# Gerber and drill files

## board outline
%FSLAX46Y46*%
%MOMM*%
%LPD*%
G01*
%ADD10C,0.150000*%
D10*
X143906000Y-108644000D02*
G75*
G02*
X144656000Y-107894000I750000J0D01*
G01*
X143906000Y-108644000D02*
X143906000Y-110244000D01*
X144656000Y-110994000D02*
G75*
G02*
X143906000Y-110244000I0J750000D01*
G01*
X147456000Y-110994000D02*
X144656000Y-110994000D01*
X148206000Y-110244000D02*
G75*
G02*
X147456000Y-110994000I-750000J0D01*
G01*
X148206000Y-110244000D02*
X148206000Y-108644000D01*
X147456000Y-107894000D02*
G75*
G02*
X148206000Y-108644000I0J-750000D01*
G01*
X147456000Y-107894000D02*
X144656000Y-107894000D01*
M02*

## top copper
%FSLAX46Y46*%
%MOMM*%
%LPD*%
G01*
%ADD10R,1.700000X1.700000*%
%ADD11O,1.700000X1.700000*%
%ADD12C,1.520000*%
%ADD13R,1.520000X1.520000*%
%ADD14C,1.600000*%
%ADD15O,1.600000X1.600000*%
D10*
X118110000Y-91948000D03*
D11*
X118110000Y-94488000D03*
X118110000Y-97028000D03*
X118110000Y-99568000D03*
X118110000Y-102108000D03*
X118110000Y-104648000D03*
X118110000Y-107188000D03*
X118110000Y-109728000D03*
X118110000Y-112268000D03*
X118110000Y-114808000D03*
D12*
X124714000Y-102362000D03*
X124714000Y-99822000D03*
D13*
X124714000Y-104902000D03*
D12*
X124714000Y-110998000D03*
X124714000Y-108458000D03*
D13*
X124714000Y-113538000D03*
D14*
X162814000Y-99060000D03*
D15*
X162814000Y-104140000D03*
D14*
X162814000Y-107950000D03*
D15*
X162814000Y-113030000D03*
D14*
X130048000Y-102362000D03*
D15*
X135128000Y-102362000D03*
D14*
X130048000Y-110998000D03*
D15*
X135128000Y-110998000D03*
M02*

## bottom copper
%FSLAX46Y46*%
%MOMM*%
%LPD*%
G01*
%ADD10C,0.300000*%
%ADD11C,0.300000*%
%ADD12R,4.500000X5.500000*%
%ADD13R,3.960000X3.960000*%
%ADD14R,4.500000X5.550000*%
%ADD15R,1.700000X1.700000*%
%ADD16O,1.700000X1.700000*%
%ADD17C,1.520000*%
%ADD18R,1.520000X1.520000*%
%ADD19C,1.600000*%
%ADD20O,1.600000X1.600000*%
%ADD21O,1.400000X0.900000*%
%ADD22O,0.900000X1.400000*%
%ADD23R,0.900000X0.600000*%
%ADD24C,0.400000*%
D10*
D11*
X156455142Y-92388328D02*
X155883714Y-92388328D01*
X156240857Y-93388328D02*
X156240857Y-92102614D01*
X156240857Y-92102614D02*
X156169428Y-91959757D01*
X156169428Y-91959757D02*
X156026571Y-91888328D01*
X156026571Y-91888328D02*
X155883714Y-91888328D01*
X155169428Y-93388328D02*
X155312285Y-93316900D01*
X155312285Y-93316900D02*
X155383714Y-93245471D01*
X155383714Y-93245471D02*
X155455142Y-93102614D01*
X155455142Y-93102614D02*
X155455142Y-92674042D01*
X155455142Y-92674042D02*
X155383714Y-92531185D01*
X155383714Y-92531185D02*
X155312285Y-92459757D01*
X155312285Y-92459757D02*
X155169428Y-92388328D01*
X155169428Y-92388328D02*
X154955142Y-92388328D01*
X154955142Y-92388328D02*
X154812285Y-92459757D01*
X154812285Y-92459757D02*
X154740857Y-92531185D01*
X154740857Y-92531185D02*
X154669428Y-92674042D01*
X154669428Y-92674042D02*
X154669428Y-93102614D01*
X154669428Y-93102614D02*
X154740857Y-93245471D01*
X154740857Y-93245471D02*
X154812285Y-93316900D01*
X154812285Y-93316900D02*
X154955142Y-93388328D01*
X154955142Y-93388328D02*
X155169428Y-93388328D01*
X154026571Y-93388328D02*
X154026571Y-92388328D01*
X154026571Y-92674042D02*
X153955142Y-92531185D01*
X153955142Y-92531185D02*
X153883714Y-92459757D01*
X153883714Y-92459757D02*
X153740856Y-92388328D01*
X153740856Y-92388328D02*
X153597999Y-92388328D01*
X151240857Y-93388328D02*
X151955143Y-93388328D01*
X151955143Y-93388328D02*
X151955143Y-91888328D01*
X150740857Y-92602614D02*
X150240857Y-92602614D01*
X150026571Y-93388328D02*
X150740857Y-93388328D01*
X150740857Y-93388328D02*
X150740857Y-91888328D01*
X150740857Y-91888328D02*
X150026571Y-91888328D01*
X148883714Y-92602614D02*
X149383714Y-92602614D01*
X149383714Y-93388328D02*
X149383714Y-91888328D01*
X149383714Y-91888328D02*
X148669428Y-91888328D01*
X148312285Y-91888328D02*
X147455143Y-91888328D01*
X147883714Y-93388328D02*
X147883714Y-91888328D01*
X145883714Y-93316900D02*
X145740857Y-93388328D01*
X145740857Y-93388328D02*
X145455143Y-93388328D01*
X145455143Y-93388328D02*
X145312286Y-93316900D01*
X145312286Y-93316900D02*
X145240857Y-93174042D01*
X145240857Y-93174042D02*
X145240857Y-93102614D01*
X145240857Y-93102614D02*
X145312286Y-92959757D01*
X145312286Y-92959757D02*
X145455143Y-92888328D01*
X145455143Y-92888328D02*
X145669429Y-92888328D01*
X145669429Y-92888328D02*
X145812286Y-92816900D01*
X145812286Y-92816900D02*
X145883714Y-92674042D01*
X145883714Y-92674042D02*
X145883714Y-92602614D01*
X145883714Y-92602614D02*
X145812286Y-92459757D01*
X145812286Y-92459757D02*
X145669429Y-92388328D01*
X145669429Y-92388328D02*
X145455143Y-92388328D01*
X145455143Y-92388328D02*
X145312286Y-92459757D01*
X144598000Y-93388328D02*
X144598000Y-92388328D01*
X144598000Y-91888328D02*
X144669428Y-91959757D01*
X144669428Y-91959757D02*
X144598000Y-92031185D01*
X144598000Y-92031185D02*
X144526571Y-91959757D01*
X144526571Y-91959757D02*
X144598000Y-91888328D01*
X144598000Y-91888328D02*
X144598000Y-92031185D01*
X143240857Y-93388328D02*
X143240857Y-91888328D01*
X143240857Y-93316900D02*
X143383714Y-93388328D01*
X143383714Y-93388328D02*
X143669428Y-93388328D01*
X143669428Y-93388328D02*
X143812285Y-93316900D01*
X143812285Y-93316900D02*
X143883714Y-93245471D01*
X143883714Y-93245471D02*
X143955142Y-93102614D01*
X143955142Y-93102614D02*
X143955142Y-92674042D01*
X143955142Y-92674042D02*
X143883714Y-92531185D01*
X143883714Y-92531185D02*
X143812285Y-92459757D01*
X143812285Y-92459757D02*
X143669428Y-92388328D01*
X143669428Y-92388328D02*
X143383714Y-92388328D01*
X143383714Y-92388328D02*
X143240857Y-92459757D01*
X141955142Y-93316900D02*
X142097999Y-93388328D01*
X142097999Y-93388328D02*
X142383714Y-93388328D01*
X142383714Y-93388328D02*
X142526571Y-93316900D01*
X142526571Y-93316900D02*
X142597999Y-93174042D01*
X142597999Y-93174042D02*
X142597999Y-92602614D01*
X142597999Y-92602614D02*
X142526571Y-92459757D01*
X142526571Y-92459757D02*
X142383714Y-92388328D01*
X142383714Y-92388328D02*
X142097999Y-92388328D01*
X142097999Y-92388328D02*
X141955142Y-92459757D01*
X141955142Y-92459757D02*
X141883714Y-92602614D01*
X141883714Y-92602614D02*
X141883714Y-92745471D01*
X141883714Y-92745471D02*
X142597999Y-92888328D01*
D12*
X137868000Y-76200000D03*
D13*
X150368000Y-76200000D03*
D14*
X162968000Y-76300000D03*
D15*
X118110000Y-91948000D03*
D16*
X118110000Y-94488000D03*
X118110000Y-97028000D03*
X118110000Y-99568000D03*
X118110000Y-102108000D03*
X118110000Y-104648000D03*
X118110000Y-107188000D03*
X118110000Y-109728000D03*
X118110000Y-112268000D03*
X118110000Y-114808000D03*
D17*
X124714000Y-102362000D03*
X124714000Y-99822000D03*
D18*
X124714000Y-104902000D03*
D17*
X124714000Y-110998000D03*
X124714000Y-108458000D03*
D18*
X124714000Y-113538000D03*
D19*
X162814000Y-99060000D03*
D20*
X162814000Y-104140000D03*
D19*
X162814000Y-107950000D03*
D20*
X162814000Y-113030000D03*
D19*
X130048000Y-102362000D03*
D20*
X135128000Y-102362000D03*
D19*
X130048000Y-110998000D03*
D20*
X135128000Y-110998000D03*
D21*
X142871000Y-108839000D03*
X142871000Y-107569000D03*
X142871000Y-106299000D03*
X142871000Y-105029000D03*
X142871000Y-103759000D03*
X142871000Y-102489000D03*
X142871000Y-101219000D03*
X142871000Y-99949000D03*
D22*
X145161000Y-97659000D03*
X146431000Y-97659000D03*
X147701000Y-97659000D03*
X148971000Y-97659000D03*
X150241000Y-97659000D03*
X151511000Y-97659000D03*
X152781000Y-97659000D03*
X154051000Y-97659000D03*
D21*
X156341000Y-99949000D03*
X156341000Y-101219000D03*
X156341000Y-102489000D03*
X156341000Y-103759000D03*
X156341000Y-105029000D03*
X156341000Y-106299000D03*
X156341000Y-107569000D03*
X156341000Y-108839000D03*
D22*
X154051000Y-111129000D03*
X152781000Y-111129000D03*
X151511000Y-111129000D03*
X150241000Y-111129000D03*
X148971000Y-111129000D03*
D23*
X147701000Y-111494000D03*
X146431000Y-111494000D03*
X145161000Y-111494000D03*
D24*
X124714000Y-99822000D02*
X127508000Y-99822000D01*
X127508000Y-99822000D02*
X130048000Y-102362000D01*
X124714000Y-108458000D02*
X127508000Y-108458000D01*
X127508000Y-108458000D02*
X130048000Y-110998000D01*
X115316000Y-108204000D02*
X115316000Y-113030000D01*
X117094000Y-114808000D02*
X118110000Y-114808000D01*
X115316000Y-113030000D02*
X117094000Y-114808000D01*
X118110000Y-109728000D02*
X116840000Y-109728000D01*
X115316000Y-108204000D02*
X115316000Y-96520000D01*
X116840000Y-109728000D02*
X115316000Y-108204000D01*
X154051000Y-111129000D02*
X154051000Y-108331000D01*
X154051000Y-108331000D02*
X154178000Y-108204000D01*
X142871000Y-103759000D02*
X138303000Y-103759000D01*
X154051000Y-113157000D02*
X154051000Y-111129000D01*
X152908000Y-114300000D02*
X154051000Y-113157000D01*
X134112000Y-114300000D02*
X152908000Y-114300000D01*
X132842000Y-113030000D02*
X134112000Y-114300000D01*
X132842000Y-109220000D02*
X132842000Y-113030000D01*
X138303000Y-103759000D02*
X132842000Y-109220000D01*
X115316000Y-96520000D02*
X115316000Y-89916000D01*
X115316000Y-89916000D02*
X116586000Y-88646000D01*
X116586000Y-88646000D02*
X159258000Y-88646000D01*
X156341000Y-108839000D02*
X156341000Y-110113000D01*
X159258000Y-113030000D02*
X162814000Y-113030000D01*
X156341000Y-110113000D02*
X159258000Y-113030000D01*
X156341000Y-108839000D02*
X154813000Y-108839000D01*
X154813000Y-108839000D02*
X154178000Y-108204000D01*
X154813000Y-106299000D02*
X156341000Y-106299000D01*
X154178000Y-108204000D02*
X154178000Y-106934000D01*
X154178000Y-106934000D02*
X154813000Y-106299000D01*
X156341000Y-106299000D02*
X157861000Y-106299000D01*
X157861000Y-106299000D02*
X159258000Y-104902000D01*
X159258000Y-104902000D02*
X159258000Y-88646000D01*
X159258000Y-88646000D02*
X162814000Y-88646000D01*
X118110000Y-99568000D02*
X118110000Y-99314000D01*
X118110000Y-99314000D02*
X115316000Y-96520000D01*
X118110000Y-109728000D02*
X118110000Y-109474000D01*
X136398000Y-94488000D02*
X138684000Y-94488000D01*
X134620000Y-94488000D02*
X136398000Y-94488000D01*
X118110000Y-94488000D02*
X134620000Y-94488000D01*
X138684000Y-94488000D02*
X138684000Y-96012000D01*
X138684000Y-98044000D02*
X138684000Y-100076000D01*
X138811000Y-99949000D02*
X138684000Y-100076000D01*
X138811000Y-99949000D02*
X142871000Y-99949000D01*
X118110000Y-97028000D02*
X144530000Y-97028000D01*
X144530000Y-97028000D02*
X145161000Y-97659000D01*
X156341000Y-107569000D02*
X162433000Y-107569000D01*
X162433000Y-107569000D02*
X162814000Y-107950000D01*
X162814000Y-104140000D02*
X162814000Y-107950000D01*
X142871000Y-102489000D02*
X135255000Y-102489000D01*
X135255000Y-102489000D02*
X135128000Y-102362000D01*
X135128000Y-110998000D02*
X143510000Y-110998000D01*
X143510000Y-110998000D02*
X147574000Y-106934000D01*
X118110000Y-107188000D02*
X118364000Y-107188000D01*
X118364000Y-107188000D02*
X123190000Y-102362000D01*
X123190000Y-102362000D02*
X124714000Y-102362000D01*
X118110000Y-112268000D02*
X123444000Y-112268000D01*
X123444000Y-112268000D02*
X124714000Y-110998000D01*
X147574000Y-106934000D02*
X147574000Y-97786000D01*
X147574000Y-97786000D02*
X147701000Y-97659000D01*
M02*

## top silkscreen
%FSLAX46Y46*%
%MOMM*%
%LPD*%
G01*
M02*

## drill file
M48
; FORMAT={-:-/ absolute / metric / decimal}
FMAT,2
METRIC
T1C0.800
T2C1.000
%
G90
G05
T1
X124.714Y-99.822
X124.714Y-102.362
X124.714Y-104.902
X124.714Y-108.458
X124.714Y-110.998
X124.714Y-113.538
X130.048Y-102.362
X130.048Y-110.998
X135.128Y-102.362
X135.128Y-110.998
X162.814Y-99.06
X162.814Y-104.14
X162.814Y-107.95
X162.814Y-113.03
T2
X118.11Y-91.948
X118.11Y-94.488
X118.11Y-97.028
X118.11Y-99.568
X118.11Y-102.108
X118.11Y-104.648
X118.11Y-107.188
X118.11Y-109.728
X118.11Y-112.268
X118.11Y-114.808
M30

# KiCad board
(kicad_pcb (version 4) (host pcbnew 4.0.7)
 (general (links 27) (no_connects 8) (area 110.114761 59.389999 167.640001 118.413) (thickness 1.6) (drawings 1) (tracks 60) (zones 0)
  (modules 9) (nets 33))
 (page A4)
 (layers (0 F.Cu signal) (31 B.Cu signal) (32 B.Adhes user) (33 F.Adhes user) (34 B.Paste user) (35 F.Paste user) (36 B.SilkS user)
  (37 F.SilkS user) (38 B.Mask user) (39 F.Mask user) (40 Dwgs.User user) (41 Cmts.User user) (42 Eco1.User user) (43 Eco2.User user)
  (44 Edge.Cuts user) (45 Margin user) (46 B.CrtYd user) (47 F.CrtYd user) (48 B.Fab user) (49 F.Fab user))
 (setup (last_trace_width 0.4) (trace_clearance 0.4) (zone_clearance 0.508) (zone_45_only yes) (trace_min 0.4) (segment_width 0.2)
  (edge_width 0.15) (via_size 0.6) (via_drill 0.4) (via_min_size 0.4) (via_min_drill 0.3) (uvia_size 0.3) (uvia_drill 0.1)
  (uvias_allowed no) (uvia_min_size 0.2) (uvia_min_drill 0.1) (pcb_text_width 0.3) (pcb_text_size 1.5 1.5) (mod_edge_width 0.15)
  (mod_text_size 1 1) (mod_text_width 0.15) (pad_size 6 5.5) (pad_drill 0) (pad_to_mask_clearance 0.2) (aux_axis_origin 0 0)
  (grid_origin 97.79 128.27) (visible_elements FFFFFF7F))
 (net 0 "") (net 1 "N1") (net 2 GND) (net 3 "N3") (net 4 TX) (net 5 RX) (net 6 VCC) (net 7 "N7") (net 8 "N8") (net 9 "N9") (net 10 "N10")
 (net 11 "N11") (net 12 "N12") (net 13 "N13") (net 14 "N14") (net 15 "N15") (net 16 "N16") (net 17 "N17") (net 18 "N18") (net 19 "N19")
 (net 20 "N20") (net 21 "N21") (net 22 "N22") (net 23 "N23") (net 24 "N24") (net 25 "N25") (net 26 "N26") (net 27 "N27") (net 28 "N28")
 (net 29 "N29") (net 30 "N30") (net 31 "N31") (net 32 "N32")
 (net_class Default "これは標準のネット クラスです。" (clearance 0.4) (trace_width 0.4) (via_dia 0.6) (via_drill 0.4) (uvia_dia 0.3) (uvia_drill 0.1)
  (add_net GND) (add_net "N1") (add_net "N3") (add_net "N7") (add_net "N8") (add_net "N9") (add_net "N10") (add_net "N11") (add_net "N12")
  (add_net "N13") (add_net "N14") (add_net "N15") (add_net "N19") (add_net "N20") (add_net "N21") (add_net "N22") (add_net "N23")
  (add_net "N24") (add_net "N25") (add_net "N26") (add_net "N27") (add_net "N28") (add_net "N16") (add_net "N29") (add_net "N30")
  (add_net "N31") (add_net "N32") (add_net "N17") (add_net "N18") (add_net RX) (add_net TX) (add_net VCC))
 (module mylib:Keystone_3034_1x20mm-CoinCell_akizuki (layer B.Cu) (at 150.368 76.2)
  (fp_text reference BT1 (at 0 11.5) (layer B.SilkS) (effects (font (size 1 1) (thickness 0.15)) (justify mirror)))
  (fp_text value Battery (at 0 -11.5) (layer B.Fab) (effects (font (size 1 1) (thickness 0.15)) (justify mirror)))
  (pad 1 smd rect (at -12.5 0) (size 4.5 5.5) (layers B.Cu B.Paste B.Mask) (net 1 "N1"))
  (pad 2 smd rect (at 0 0) (size 3.96 3.96) (layers B.Cu B.Paste B.Mask) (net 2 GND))
  (pad 1 smd rect (at 12.6 0.1) (size 4.5 5.55) (layers B.Cu B.Paste B.Mask) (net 1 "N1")))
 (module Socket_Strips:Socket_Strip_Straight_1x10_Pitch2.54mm (layer B.Cu) (at 118.11 91.948 180)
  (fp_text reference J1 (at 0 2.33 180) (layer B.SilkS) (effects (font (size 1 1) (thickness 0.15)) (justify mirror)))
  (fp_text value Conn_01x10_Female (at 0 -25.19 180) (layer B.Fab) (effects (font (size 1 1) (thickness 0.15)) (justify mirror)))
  (pad 1 thru_hole rect (at 0 0 180) (size 1.7 1.7) (drill 1) (layers *.Cu *.Mask) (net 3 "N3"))
  (pad 2 thru_hole oval (at 0 -2.54 180) (size 1.7 1.7) (drill 1) (layers *.Cu *.Mask) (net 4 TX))
  (pad 3 thru_hole oval (at 0 -5.08 180) (size 1.7 1.7) (drill 1) (layers *.Cu *.Mask) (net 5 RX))
  (pad 4 thru_hole oval (at 0 -7.62 180) (size 1.7 1.7) (drill 1) (layers *.Cu *.Mask) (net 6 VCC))
  (pad 5 thru_hole oval (at 0 -10.16 180) (size 1.7 1.7) (drill 1) (layers *.Cu *.Mask) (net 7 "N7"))
  (pad 6 thru_hole oval (at 0 -12.7 180) (size 1.7 1.7) (drill 1) (layers *.Cu *.Mask) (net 2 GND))
  (pad 7 thru_hole oval (at 0 -15.24 180) (size 1.7 1.7) (drill 1) (layers *.Cu *.Mask) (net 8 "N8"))
  (pad 8 thru_hole oval (at 0 -17.78 180) (size 1.7 1.7) (drill 1) (layers *.Cu *.Mask) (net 6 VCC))
  (pad 9 thru_hole oval (at 0 -20.32 180) (size 1.7 1.7) (drill 1) (layers *.Cu *.Mask) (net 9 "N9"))
  (pad 10 thru_hole oval (at 0 -22.86 180) (size 1.7 1.7) (drill 1) (layers *.Cu *.Mask) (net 6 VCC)))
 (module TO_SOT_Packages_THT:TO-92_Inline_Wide (layer B.Cu) (at 124.714 104.902 90)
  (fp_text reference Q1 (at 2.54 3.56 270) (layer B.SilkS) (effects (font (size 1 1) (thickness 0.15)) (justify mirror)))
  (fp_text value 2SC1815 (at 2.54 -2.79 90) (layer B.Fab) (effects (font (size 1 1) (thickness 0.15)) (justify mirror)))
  (pad 2 thru_hole circle (at 2.54 0) (size 1.52 1.52) (drill 0.8) (layers *.Cu *.Mask) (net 8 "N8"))
  (pad 3 thru_hole circle (at 5.08 0) (size 1.52 1.52) (drill 0.8) (layers *.Cu *.Mask) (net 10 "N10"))
  (pad 1 thru_hole rect (at 0 0) (size 1.52 1.52) (drill 0.8) (layers *.Cu *.Mask) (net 2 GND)))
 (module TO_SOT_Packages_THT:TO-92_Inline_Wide (layer B.Cu) (at 124.714 113.538 90)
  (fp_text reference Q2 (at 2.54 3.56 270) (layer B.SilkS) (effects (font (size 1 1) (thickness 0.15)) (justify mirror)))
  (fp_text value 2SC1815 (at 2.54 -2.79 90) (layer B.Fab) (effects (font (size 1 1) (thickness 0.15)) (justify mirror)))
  (pad 2 thru_hole circle (at 2.54 0) (size 1.52 1.52) (drill 0.8) (layers *.Cu *.Mask) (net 9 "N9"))
  (pad 3 thru_hole circle (at 5.08 0) (size 1.52 1.52) (drill 0.8) (layers *.Cu *.Mask) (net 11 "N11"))
  (pad 1 thru_hole rect (at 0 0) (size 1.52 1.52) (drill 0.8) (layers *.Cu *.Mask) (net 2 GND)))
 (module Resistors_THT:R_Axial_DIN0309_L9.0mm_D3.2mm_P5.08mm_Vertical (layer B.Cu) (at 162.814 99.06 270)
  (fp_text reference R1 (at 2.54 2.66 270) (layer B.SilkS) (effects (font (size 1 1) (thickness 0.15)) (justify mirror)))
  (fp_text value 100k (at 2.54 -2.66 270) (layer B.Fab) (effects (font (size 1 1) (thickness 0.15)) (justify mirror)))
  (pad 1 thru_hole circle (at 0 0 270) (size 1.6 1.6) (drill 0.8) (layers *.Cu *.Mask) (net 2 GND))
  (pad 2 thru_hole oval (at 5.08 0 270) (size 1.6 1.6) (drill 0.8) (layers *.Cu *.Mask) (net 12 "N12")))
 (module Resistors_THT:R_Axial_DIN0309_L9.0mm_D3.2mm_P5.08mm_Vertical (layer B.Cu) (at 162.814 107.95 270)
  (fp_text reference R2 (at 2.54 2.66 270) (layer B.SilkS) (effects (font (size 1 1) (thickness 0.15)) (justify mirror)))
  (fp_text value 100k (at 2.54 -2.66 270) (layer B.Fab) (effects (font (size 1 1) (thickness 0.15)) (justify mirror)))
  (pad 1 thru_hole circle (at 0 0 270) (size 1.6 1.6) (drill 0.8) (layers *.Cu *.Mask) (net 12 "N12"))
  (pad 2 thru_hole oval (at 5.08 0 270) (size 1.6 1.6) (drill 0.8) (layers *.Cu *.Mask) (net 6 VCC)))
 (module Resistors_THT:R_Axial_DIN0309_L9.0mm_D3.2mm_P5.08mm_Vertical (layer B.Cu) (at 130.048 102.362)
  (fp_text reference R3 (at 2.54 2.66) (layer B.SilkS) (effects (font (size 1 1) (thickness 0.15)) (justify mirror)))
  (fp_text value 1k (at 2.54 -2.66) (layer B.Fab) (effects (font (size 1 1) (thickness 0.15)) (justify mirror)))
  (pad 1 thru_hole circle (at 0 0) (size 1.6 1.6) (drill 0.8) (layers *.Cu *.Mask) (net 10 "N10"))
  (pad 2 thru_hole oval (at 5.08 0) (size 1.6 1.6) (drill 0.8) (layers *.Cu *.Mask) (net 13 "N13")))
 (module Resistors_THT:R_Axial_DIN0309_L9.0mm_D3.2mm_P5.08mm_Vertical (layer B.Cu) (at 130.048 110.998)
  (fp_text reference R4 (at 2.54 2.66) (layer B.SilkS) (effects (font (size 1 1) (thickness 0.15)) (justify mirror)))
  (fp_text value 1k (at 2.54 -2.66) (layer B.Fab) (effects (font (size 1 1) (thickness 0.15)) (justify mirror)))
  (pad 1 thru_hole circle (at 0 0) (size 1.6 1.6) (drill 0.8) (layers *.Cu *.Mask) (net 11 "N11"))
  (pad 2 thru_hole oval (at 5.08 0) (size 1.6 1.6) (drill 0.8) (layers *.Cu *.Mask) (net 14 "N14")))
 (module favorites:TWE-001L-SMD (layer B.Cu) (at 149.606 104.394)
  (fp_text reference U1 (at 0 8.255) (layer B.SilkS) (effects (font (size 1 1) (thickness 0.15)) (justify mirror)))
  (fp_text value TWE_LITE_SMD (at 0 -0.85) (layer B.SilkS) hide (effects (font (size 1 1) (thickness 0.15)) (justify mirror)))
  (fp_arc (start -4.95 4.25) (end -4.95 3.5) (angle -90) (layer Edge.Cuts) (width 0.15))
  (fp_line (start -5.7 4.25) (end -5.7 5.85) (layer Edge.Cuts) (width 0.15))
  (fp_arc (start -4.95 5.85) (end -5.7 5.85) (angle -90) (layer Edge.Cuts) (width 0.15))
  (fp_line (start -2.15 6.6) (end -4.95 6.6) (layer Edge.Cuts) (width 0.15))
  (fp_arc (start -2.15 5.85) (end -2.15 6.6) (angle -90) (layer Edge.Cuts) (width 0.15))
  (fp_line (start -1.4 5.85) (end -1.4 4.25) (layer Edge.Cuts) (width 0.15))
  (fp_arc (start -2.15 4.25) (end -1.4 4.25) (angle -90) (layer Edge.Cuts) (width 0.15))
  (fp_line (start -2.15 3.5) (end -4.95 3.5) (layer Edge.Cuts) (width 0.15))
  (pad 1 smd oval (at -6.735 4.445 270) (size 0.9 1.4) (layers B.Cu B.Paste B.Mask) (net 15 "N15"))
  (pad 2 smd oval (at -6.735 3.175 270) (size 0.9 1.4) (layers B.Cu B.Paste B.Mask) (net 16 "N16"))
  (pad 3 smd oval (at -6.735 1.905 270) (size 0.9 1.4) (layers B.Cu B.Paste B.Mask) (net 14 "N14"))
  (pad 4 smd oval (at -6.735 0.635 270) (size 0.9 1.4) (layers B.Cu B.Paste B.Mask) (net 13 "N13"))
  (pad 5 smd oval (at -6.735 -0.635 270) (size 0.9 1.4) (layers B.Cu B.Paste B.Mask) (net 6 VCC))
  (pad 6 smd oval (at -6.735 -1.905 270) (size 0.9 1.4) (layers B.Cu B.Paste B.Mask) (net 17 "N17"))
  (pad 7 smd oval (at -6.735 -3.175 270) (size 0.9 1.4) (layers B.Cu B.Paste B.Mask) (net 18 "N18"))
  (pad 8 smd oval (at -6.735 -4.445 270) (size 0.9 1.4) (layers B.Cu B.Paste B.Mask) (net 4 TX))
  (pad 9 smd oval (at -4.445 -6.735) (size 0.9 1.4) (layers B.Cu B.Paste B.Mask) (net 5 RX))
  (pad 10 smd oval (at -3.175 -6.735) (size 0.9 1.4) (layers B.Cu B.Paste B.Mask) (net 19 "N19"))
  (pad 11 smd oval (at -1.905 -6.735) (size 0.9 1.4) (layers B.Cu B.Paste B.Mask) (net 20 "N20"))
  (pad 12 smd oval (at -0.635 -6.735) (size 0.9 1.4) (layers B.Cu B.Paste B.Mask) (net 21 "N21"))
  (pad 13 smd oval (at 0.635 -6.735) (size 0.9 1.4) (layers B.Cu B.Paste B.Mask) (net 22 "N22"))
  (pad 14 smd oval (at 1.905 -6.735) (size 0.9 1.4) (layers B.Cu B.Paste B.Mask) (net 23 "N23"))
  (pad 15 smd oval (at 3.175 -6.735) (size 0.9 1.4) (layers B.Cu B.Paste B.Mask) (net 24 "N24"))
  (pad 16 smd oval (at 4.445 -6.735) (size 0.9 1.4) (layers B.Cu B.Paste B.Mask) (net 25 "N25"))
  (pad 17 smd oval (at 6.735 -4.445 270) (size 0.9 1.4) (layers B.Cu B.Paste B.Mask) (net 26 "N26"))
  (pad 18 smd oval (at 6.735 -3.175 270) (size 0.9 1.4) (layers B.Cu B.Paste B.Mask) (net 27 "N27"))
  (pad 19 smd oval (at 6.735 -1.905 270) (size 0.9 1.4) (layers B.Cu B.Paste B.Mask) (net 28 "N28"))
  (pad 20 smd oval (at 6.735 -0.635 270) (size 0.9 1.4) (layers B.Cu B.Paste B.Mask) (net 2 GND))
  (pad 21 smd oval (at 6.735 0.635 270) (size 0.9 1.4) (layers B.Cu B.Paste B.Mask) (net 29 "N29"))
  (pad 22 smd oval (at 6.735 1.905 270) (size 0.9 1.4) (layers B.Cu B.Paste B.Mask) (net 6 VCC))
  (pad 23 smd oval (at 6.735 3.175 270) (size 0.9 1.4) (layers B.Cu B.Paste B.Mask) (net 12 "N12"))
  (pad 24 smd oval (at 6.735 4.445 270) (size 0.9 1.4) (layers B.Cu B.Paste B.Mask) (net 6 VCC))
  (pad 25 smd oval (at 4.445 6.735) (size 0.9 1.4) (layers B.Cu B.Paste B.Mask) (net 6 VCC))
  (pad 26 smd oval (at 3.175 6.735) (size 0.9 1.4) (layers B.Cu B.Paste B.Mask) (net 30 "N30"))
  (pad 27 smd oval (at 1.905 6.735) (size 0.9 1.4) (layers B.Cu B.Paste B.Mask) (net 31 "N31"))
  (pad 28 smd oval (at 0.635 6.735) (size 0.9 1.4) (layers B.Cu B.Paste B.Mask) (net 2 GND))
  (pad 29 smd oval (at -0.635 6.735) (size 0.9 1.4) (layers B.Cu B.Paste B.Mask) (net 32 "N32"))
  (pad 30 smd rect (at -1.905 7.1) (size 0.9 0.6) (layers B.Cu B.Paste B.Mask) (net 2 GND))
  (pad 31 smd rect (at -3.175 7.1) (size 0.9 0.6) (layers B.Cu B.Paste B.Mask) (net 2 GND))
  (pad 32 smd rect (at -4.445 7.1) (size 0.9 0.6) (layers B.Cu B.Paste B.Mask) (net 2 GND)))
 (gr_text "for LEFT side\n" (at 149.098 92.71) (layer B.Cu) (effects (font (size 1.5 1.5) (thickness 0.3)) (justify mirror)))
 (segment (start 124.714 99.822) (end 127.508 99.822) (width 0.4) (layer B.Cu) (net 10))
 (segment (start 127.508 99.822) (end 130.048 102.362) (width 0.4) (layer B.Cu) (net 10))
 (segment (start 124.714 108.458) (end 127.508 108.458) (width 0.4) (layer B.Cu) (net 11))
 (segment (start 127.508 108.458) (end 130.048 110.998) (width 0.4) (layer B.Cu) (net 11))
 (segment (start 115.316 108.204) (end 115.316 113.03) (width 0.4) (layer B.Cu) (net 6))
 (segment (start 117.094 114.808) (end 118.11 114.808) (width 0.4) (layer B.Cu) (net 6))
 (segment (start 115.316 113.03) (end 117.094 114.808) (width 0.4) (layer B.Cu) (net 6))
 (segment (start 118.11 109.728) (end 116.84 109.728) (width 0.4) (layer B.Cu) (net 6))
 (segment (start 115.316 108.204) (end 115.316 96.52) (width 0.4) (layer B.Cu) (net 6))
 (segment (start 116.84 109.728) (end 115.316 108.204) (width 0.4) (layer B.Cu) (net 6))
 (segment (start 154.051 111.129) (end 154.051 108.331) (width 0.4) (layer B.Cu) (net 6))
 (segment (start 154.051 108.331) (end 154.178 108.204) (width 0.4) (layer B.Cu) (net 6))
 (segment (start 142.871 103.759) (end 138.303 103.759) (width 0.4) (layer B.Cu) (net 6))
 (segment (start 154.051 113.157) (end 154.051 111.129) (width 0.4) (layer B.Cu) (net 6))
 (segment (start 152.908 114.3) (end 154.051 113.157) (width 0.4) (layer B.Cu) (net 6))
 (segment (start 134.112 114.3) (end 152.908 114.3) (width 0.4) (layer B.Cu) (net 6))
 (segment (start 132.842 113.03) (end 134.112 114.3) (width 0.4) (layer B.Cu) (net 6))
 (segment (start 132.842 109.22) (end 132.842 113.03) (width 0.4) (layer B.Cu) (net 6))
 (segment (start 138.303 103.759) (end 132.842 109.22) (width 0.4) (layer B.Cu) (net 6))
 (segment (start 115.316 96.52) (end 115.316 89.916) (width 0.4) (layer B.Cu) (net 6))
 (segment (start 115.316 89.916) (end 116.586 88.646) (width 0.4) (layer B.Cu) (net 6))
 (segment (start 116.586 88.646) (end 159.258 88.646) (width 0.4) (layer B.Cu) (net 6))
 (segment (start 156.341 108.839) (end 156.341 110.113) (width 0.4) (layer B.Cu) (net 6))
 (segment (start 159.258 113.03) (end 162.814 113.03) (width 0.4) (layer B.Cu) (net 6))
 (segment (start 156.341 110.113) (end 159.258 113.03) (width 0.4) (layer B.Cu) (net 6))
 (segment (start 156.341 108.839) (end 154.813 108.839) (width 0.4) (layer B.Cu) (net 6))
 (segment (start 154.813 108.839) (end 154.178 108.204) (width 0.4) (layer B.Cu) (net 6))
 (segment (start 154.813 106.299) (end 156.341 106.299) (width 0.4) (layer B.Cu) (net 6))
 (segment (start 154.178 108.204) (end 154.178 106.934) (width 0.4) (layer B.Cu) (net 6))
 (segment (start 154.178 106.934) (end 154.813 106.299) (width 0.4) (layer B.Cu) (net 6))
 (segment (start 156.341 106.299) (end 157.861 106.299) (width 0.4) (layer B.Cu) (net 6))
 (segment (start 157.861 106.299) (end 159.258 104.902) (width 0.4) (layer B.Cu) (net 6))
 (segment (start 159.258 104.902) (end 159.258 88.646) (width 0.4) (layer B.Cu) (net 6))
 (segment (start 159.258 88.646) (end 162.814 88.646) (width 0.4) (layer B.Cu) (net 6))
 (segment (start 118.11 99.568) (end 118.11 99.314) (width 0.4) (layer B.Cu) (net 6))
 (segment (start 118.11 99.314) (end 115.316 96.52) (width 0.4) (layer B.Cu) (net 6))
 (segment (start 118.11 109.728) (end 118.11 109.474) (width 0.4) (layer B.Cu) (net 6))
 (segment (start 136.398 94.488) (end 138.684 94.488) (width 0.4) (layer B.Cu) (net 4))
 (segment (start 134.62 94.488) (end 136.398 94.488) (width 0.4) (layer B.Cu) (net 4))
 (segment (start 118.11 94.488) (end 134.62 94.488) (width 0.4) (layer B.Cu) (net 4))
 (segment (start 138.684 94.488) (end 138.684 96.012) (width 0.4) (layer B.Cu) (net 4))
 (segment (start 138.684 98.044) (end 138.684 100.076) (width 0.4) (layer B.Cu) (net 4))
 (segment (start 138.811 99.949) (end 138.684 100.076) (width 0.4) (layer B.Cu) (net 4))
 (segment (start 138.811 99.949) (end 142.871 99.949) (width 0.4) (layer B.Cu) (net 4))
 (segment (start 118.11 97.028) (end 144.53 97.028) (width 0.4) (layer B.Cu) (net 5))
 (segment (start 144.53 97.028) (end 145.161 97.659) (width 0.4) (layer B.Cu) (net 5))
 (segment (start 156.341 107.569) (end 162.433 107.569) (width 0.4) (layer B.Cu) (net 12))
 (segment (start 162.433 107.569) (end 162.814 107.95) (width 0.4) (layer B.Cu) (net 12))
 (segment (start 162.814 104.14) (end 162.814 107.95) (width 0.4) (layer B.Cu) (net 12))
 (segment (start 142.871 102.489) (end 135.255 102.489) (width 0.4) (layer B.Cu) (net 13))
 (segment (start 135.255 102.489) (end 135.128 102.362) (width 0.4) (layer B.Cu) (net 13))
 (segment (start 135.128 110.998) (end 143.51 110.998) (width 0.4) (layer B.Cu) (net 14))
 (segment (start 143.51 110.998) (end 147.574 106.934) (width 0.4) (layer B.Cu) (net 14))
 (segment (start 118.11 107.188) (end 118.364 107.188) (width 0.4) (layer B.Cu) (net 8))
 (segment (start 118.364 107.188) (end 123.19 102.362) (width 0.4) (layer B.Cu) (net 8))
 (segment (start 123.19 102.362) (end 124.714 102.362) (width 0.4) (layer B.Cu) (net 8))
 (segment (start 118.11 112.268) (end 123.444 112.268) (width 0.4) (layer B.Cu) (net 9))
 (segment (start 123.444 112.268) (end 124.714 110.998) (width 0.4) (layer B.Cu) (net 9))
 (segment (start 147.574 106.934) (end 147.574 97.786) (width 0.4) (layer B.Cu) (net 20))
 (segment (start 147.574 97.786) (end 147.701 97.659) (width 0.4) (layer B.Cu) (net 20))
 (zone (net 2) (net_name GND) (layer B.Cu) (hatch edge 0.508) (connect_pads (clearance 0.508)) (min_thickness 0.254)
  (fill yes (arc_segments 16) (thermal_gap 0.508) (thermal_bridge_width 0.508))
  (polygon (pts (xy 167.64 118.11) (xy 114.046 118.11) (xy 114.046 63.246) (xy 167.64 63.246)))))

